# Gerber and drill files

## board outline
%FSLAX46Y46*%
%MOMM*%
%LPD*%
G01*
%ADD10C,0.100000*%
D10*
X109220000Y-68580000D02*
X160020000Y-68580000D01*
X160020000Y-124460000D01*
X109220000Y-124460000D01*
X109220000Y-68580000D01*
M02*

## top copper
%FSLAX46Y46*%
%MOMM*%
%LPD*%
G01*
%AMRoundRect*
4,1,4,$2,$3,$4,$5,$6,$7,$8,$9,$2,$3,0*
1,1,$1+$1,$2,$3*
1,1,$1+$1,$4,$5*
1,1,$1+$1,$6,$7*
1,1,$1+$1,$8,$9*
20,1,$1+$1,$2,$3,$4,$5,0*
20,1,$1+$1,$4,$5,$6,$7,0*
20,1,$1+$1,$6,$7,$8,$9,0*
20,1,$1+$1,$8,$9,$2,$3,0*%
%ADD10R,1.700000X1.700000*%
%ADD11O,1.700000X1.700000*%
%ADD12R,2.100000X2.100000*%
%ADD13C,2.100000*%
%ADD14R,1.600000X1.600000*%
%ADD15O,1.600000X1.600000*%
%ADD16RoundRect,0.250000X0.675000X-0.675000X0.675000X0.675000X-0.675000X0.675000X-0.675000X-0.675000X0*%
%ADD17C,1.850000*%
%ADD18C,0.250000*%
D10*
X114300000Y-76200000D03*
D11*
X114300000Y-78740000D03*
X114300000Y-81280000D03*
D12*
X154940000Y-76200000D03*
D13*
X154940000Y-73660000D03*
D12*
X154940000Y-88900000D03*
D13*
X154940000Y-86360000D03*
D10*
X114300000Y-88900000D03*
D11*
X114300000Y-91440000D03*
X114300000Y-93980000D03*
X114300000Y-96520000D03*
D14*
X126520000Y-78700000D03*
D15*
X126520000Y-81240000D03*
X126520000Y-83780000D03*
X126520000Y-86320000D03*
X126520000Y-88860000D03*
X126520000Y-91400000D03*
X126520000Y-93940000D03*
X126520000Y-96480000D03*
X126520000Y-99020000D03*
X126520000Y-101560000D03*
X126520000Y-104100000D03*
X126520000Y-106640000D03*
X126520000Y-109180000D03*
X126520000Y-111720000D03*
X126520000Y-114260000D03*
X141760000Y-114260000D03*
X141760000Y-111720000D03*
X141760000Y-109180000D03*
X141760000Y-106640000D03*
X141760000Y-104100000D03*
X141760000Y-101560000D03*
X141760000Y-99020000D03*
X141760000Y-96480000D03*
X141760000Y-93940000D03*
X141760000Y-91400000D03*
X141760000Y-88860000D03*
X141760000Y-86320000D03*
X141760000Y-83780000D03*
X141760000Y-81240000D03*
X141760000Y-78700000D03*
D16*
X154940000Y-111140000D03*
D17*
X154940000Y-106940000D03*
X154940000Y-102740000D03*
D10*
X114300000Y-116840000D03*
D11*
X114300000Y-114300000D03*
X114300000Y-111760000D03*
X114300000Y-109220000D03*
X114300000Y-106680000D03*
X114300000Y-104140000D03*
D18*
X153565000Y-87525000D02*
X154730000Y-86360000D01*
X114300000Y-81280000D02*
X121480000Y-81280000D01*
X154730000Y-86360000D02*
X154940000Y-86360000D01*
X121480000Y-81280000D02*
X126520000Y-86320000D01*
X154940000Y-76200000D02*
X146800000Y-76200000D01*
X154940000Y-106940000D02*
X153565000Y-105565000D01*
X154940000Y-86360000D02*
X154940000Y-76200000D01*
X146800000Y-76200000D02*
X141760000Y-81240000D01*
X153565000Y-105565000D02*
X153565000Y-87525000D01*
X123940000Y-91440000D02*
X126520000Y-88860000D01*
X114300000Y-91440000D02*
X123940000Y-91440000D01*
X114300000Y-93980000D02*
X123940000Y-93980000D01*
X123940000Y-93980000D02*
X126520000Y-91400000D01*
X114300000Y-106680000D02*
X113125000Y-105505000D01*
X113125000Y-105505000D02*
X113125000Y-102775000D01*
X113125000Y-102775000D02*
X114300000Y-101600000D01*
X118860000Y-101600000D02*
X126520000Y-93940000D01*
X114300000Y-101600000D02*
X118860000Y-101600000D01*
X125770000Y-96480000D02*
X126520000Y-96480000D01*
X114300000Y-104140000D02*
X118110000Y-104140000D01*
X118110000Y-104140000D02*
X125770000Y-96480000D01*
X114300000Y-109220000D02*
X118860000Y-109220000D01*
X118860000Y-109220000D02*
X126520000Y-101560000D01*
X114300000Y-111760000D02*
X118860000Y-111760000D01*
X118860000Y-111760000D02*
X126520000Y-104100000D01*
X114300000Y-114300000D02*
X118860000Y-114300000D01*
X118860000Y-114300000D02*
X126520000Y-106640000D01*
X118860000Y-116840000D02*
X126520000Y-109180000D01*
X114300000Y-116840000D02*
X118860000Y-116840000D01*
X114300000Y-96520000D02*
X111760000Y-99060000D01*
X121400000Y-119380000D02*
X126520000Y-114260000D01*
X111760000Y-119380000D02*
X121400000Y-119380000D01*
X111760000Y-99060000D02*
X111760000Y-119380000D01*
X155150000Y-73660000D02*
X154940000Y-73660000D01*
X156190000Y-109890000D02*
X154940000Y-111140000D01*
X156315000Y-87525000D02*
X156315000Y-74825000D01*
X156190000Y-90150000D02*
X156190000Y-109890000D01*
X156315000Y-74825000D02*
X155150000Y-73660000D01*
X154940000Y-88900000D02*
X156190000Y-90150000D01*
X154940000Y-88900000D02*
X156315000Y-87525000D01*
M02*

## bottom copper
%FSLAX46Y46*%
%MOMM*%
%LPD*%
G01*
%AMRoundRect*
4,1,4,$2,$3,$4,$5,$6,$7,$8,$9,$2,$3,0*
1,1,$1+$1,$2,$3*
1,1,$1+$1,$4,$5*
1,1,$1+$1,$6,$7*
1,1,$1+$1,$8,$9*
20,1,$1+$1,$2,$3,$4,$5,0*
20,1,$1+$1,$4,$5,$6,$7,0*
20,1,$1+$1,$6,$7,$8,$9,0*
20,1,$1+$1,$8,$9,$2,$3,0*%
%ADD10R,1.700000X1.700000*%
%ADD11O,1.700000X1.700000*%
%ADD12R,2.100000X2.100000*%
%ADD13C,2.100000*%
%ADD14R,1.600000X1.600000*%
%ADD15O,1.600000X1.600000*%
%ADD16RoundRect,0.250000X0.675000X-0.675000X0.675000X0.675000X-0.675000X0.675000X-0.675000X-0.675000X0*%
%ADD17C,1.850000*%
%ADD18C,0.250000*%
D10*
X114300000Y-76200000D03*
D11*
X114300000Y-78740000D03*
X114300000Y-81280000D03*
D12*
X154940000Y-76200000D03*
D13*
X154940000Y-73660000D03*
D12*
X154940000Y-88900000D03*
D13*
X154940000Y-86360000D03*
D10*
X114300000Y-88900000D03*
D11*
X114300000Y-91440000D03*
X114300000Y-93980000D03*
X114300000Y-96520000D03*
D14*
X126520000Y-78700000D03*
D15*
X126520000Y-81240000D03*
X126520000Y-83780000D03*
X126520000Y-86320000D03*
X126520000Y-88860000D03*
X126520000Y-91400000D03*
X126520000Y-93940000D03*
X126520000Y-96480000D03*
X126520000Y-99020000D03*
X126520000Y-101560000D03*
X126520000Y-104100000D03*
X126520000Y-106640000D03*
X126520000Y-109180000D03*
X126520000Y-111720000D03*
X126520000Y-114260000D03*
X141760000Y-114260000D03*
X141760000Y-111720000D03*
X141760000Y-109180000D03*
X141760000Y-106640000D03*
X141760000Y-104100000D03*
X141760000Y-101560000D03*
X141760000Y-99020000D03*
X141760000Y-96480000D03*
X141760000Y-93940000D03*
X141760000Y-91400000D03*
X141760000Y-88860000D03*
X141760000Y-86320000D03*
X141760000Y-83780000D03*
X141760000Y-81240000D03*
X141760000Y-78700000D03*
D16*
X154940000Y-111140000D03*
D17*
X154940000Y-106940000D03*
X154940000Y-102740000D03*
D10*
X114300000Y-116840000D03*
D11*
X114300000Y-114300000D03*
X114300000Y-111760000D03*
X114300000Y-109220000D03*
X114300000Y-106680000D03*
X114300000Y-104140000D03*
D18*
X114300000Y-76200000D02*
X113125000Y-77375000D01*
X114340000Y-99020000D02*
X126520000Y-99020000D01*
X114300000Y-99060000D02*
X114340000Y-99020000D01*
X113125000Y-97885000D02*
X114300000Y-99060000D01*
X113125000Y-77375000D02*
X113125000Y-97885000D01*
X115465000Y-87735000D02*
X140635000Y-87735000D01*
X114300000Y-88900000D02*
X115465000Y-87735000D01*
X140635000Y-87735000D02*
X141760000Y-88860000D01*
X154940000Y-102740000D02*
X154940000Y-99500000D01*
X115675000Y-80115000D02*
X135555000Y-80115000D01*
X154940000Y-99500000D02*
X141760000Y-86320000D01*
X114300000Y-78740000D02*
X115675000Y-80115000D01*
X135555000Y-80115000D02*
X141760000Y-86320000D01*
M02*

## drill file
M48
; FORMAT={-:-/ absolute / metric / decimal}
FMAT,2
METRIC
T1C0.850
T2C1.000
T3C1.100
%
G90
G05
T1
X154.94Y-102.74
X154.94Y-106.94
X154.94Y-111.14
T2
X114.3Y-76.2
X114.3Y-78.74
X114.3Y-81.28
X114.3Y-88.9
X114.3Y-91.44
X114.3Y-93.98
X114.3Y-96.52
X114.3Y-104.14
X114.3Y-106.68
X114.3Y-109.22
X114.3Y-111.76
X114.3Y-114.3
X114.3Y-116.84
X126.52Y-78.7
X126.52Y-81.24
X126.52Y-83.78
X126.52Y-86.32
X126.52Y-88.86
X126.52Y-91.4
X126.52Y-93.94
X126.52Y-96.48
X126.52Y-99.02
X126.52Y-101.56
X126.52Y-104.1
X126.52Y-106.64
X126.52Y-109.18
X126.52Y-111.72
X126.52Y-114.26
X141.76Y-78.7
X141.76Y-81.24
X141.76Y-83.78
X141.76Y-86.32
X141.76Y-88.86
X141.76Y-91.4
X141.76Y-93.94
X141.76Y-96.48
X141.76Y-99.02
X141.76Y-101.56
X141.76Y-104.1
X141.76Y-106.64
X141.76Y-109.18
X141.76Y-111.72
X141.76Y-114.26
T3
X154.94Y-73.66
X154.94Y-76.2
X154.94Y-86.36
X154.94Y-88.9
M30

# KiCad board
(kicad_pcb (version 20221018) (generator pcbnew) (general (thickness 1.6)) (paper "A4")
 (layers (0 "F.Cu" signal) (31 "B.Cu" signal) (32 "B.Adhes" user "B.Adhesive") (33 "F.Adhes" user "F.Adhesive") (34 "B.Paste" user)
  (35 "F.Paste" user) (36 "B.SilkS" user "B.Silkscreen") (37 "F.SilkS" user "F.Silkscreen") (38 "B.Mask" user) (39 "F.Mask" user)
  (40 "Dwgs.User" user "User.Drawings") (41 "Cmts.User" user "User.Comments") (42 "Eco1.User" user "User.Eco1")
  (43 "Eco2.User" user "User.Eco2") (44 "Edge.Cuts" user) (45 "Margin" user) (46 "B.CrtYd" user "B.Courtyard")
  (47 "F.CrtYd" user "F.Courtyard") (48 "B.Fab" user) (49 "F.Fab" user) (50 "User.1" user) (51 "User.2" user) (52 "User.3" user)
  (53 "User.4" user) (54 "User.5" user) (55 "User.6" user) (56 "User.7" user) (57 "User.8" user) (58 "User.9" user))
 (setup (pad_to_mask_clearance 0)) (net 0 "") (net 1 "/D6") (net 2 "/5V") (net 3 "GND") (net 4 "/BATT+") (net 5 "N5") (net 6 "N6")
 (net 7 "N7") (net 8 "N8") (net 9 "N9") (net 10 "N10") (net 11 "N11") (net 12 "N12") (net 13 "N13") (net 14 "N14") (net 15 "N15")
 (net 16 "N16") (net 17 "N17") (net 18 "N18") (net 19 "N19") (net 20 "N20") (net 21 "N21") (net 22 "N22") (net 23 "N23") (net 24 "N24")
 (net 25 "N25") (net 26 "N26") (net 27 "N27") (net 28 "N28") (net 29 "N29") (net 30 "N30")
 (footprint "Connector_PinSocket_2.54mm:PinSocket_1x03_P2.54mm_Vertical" (layer "F.Cu") (at 114.3 76.2)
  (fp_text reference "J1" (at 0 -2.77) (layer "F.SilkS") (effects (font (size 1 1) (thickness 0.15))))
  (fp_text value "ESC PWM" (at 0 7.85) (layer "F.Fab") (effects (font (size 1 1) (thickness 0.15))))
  (pad "1" thru_hole rect (at 0 0) (size 1.7 1.7) (drill 1) (layers "*.Cu" "*.Mask") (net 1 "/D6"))
  (pad "2" thru_hole oval (at 0 2.54) (size 1.7 1.7) (drill 1) (layers "*.Cu" "*.Mask") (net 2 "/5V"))
  (pad "3" thru_hole oval (at 0 5.08) (size 1.7 1.7) (drill 1) (layers "*.Cu" "*.Mask") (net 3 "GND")))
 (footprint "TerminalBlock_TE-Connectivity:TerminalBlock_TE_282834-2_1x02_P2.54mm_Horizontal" (layer "F.Cu") (at 154.94 76.2 90)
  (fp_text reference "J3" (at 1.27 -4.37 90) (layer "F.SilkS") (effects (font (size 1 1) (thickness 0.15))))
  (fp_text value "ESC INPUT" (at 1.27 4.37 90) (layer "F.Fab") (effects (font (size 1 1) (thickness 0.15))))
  (pad "1" thru_hole rect (at 0 0 90) (size 2.1 2.1) (drill 1.1) (layers "*.Cu" "*.Mask") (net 3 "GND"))
  (pad "2" thru_hole circle (at 2.54 0 90) (size 2.1 2.1) (drill 1.1) (layers "*.Cu" "*.Mask") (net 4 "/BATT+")))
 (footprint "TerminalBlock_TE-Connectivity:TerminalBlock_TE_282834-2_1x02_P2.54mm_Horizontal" (layer "F.Cu") (at 154.94 88.9 90)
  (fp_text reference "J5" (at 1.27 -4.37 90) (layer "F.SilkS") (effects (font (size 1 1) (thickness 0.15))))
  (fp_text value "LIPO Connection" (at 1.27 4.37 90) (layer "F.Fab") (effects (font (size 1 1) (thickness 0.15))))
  (pad "1" thru_hole rect (at 0 0 90) (size 2.1 2.1) (drill 1.1) (layers "*.Cu" "*.Mask") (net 4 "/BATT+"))
  (pad "2" thru_hole circle (at 2.54 0 90) (size 2.1 2.1) (drill 1.1) (layers "*.Cu" "*.Mask") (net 3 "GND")))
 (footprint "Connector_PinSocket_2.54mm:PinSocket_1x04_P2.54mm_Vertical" (layer "F.Cu") (at 114.3 88.9)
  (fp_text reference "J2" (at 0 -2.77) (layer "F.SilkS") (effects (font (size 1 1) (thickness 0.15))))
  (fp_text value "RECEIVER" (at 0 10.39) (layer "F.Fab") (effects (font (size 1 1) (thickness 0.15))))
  (pad "1" thru_hole rect (at 0 0) (size 1.7 1.7) (drill 1) (layers "*.Cu" "*.Mask") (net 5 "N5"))
  (pad "2" thru_hole oval (at 0 2.54) (size 1.7 1.7) (drill 1) (layers "*.Cu" "*.Mask") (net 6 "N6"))
  (pad "3" thru_hole oval (at 0 5.08) (size 1.7 1.7) (drill 1) (layers "*.Cu" "*.Mask") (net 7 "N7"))
  (pad "4" thru_hole oval (at 0 7.62) (size 1.7 1.7) (drill 1) (layers "*.Cu" "*.Mask") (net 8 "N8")))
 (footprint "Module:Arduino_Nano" (layer "F.Cu") (at 126.52 78.7)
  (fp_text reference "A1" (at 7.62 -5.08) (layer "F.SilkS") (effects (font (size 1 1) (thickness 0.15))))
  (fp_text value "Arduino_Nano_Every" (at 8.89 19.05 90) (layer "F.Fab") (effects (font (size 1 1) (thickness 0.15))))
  (pad "1" thru_hole rect (at 0 0) (size 1.6 1.6) (drill 1) (layers "*.Cu" "*.Mask") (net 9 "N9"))
  (pad "2" thru_hole oval (at 0 2.54) (size 1.6 1.6) (drill 1) (layers "*.Cu" "*.Mask") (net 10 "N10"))
  (pad "3" thru_hole oval (at 0 5.08) (size 1.6 1.6) (drill 1) (layers "*.Cu" "*.Mask") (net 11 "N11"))
  (pad "4" thru_hole oval (at 0 7.62) (size 1.6 1.6) (drill 1) (layers "*.Cu" "*.Mask") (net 3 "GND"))
  (pad "5" thru_hole oval (at 0 10.16) (size 1.6 1.6) (drill 1) (layers "*.Cu" "*.Mask") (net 6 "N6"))
  (pad "6" thru_hole oval (at 0 12.7) (size 1.6 1.6) (drill 1) (layers "*.Cu" "*.Mask") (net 7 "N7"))
  (pad "7" thru_hole oval (at 0 15.24) (size 1.6 1.6) (drill 1) (layers "*.Cu" "*.Mask") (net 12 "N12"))
  (pad "8" thru_hole oval (at 0 17.78) (size 1.6 1.6) (drill 1) (layers "*.Cu" "*.Mask") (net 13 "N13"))
  (pad "9" thru_hole oval (at 0 20.32) (size 1.6 1.6) (drill 1) (layers "*.Cu" "*.Mask") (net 1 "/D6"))
  (pad "10" thru_hole oval (at 0 22.86) (size 1.6 1.6) (drill 1) (layers "*.Cu" "*.Mask") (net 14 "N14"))
  (pad "11" thru_hole oval (at 0 25.4) (size 1.6 1.6) (drill 1) (layers "*.Cu" "*.Mask") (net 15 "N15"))
  (pad "12" thru_hole oval (at 0 27.94) (size 1.6 1.6) (drill 1) (layers "*.Cu" "*.Mask") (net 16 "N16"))
  (pad "13" thru_hole oval (at 0 30.48) (size 1.6 1.6) (drill 1) (layers "*.Cu" "*.Mask") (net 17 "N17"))
  (pad "14" thru_hole oval (at 0 33.02) (size 1.6 1.6) (drill 1) (layers "*.Cu" "*.Mask") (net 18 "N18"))
  (pad "15" thru_hole oval (at 0 35.56) (size 1.6 1.6) (drill 1) (layers "*.Cu" "*.Mask") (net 8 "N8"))
  (pad "16" thru_hole oval (at 15.24 35.56) (size 1.6 1.6) (drill 1) (layers "*.Cu" "*.Mask") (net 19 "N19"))
  (pad "17" thru_hole oval (at 15.24 33.02) (size 1.6 1.6) (drill 1) (layers "*.Cu" "*.Mask") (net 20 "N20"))
  (pad "18" thru_hole oval (at 15.24 30.48) (size 1.6 1.6) (drill 1) (layers "*.Cu" "*.Mask") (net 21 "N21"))
  (pad "19" thru_hole oval (at 15.24 27.94) (size 1.6 1.6) (drill 1) (layers "*.Cu" "*.Mask") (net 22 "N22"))
  (pad "20" thru_hole oval (at 15.24 25.4) (size 1.6 1.6) (drill 1) (layers "*.Cu" "*.Mask") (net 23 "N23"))
  (pad "21" thru_hole oval (at 15.24 22.86) (size 1.6 1.6) (drill 1) (layers "*.Cu" "*.Mask") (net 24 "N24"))
  (pad "22" thru_hole oval (at 15.24 20.32) (size 1.6 1.6) (drill 1) (layers "*.Cu" "*.Mask") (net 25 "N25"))
  (pad "23" thru_hole oval (at 15.24 17.78) (size 1.6 1.6) (drill 1) (layers "*.Cu" "*.Mask") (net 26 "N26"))
  (pad "24" thru_hole oval (at 15.24 15.24) (size 1.6 1.6) (drill 1) (layers "*.Cu" "*.Mask") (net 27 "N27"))
  (pad "25" thru_hole oval (at 15.24 12.7) (size 1.6 1.6) (drill 1) (layers "*.Cu" "*.Mask") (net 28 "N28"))
  (pad "26" thru_hole oval (at 15.24 10.16) (size 1.6 1.6) (drill 1) (layers "*.Cu" "*.Mask") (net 5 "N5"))
  (pad "27" thru_hole oval (at 15.24 7.62) (size 1.6 1.6) (drill 1) (layers "*.Cu" "*.Mask") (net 2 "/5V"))
  (pad "28" thru_hole oval (at 15.24 5.08) (size 1.6 1.6) (drill 1) (layers "*.Cu" "*.Mask") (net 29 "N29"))
  (pad "29" thru_hole oval (at 15.24 2.54) (size 1.6 1.6) (drill 1) (layers "*.Cu" "*.Mask") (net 3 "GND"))
  (pad "30" thru_hole oval (at 15.24 0) (size 1.6 1.6) (drill 1) (layers "*.Cu" "*.Mask") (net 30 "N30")))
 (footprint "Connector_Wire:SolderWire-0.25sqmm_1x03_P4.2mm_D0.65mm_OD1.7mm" (layer "F.Cu") (at 154.94 111.14 90)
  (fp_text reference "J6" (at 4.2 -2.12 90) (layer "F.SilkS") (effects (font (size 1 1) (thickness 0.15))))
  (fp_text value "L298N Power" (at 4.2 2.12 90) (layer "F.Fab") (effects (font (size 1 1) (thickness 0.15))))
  (pad "1" thru_hole roundrect (at 0 0 90) (size 1.85 1.85) (drill 0.85) (layers "*.Cu" "*.Mask") (roundrect_rratio 0.1351351351)
   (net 4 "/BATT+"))
  (pad "2" thru_hole circle (at 4.2 0 90) (size 1.85 1.85) (drill 0.85) (layers "*.Cu" "*.Mask") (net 3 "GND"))
  (pad "3" thru_hole circle (at 8.4 0 90) (size 1.85 1.85) (drill 0.85) (layers "*.Cu" "*.Mask") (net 2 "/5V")))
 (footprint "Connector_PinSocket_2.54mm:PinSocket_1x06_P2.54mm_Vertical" (layer "F.Cu") (at 114.3 116.84 180)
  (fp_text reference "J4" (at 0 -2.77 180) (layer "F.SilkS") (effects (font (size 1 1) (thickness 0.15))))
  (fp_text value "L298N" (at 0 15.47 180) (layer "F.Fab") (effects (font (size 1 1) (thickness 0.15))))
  (pad "1" thru_hole rect (at 0 0 180) (size 1.7 1.7) (drill 1) (layers "*.Cu" "*.Mask") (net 17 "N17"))
  (pad "2" thru_hole oval (at 0 2.54 180) (size 1.7 1.7) (drill 1) (layers "*.Cu" "*.Mask") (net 16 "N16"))
  (pad "3" thru_hole oval (at 0 5.08 180) (size 1.7 1.7) (drill 1) (layers "*.Cu" "*.Mask") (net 15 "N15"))
  (pad "4" thru_hole oval (at 0 7.62 180) (size 1.7 1.7) (drill 1) (layers "*.Cu" "*.Mask") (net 14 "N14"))
  (pad "5" thru_hole oval (at 0 10.16 180) (size 1.7 1.7) (drill 1) (layers "*.Cu" "*.Mask") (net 12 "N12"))
  (pad "6" thru_hole oval (at 0 12.7 180) (size 1.7 1.7) (drill 1) (layers "*.Cu" "*.Mask") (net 13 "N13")))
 (gr_rect (start 109.22 68.58) (end 160.02 124.46) (stroke (width 0.1) (type default)) (fill none) (layer "Edge.Cuts"))
 (segment (start 153.565 87.525) (end 154.73 86.36) (width 0.25) (layer "F.Cu") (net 3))
 (segment (start 114.3 81.28) (end 121.48 81.28) (width 0.25) (layer "F.Cu") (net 3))
 (segment (start 154.73 86.36) (end 154.94 86.36) (width 0.25) (layer "F.Cu") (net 3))
 (segment (start 121.48 81.28) (end 126.52 86.32) (width 0.25) (layer "F.Cu") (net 3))
 (segment (start 154.94 76.2) (end 146.8 76.2) (width 0.25) (layer "F.Cu") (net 3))
 (segment (start 154.94 106.94) (end 153.565 105.565) (width 0.25) (layer "F.Cu") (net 3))
 (segment (start 154.94 86.36) (end 154.94 76.2) (width 0.25) (layer "F.Cu") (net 3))
 (segment (start 146.8 76.2) (end 141.76 81.24) (width 0.25) (layer "F.Cu") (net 3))
 (segment (start 153.565 105.565) (end 153.565 87.525) (width 0.25) (layer "F.Cu") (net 3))
 (segment (start 123.94 91.44) (end 126.52 88.86) (width 0.25) (layer "F.Cu") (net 6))
 (segment (start 114.3 91.44) (end 123.94 91.44) (width 0.25) (layer "F.Cu") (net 6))
 (segment (start 114.3 93.98) (end 123.94 93.98) (width 0.25) (layer "F.Cu") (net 7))
 (segment (start 123.94 93.98) (end 126.52 91.4) (width 0.25) (layer "F.Cu") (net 7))
 (segment (start 114.3 106.68) (end 113.125 105.505) (width 0.25) (layer "F.Cu") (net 12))
 (segment (start 113.125 105.505) (end 113.125 102.775) (width 0.25) (layer "F.Cu") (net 12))
 (segment (start 113.125 102.775) (end 114.3 101.6) (width 0.25) (layer "F.Cu") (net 12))
 (segment (start 118.86 101.6) (end 126.52 93.94) (width 0.25) (layer "F.Cu") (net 12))
 (segment (start 114.3 101.6) (end 118.86 101.6) (width 0.25) (layer "F.Cu") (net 12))
 (segment (start 125.77 96.48) (end 126.52 96.48) (width 0.25) (layer "F.Cu") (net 13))
 (segment (start 114.3 104.14) (end 118.11 104.14) (width 0.25) (layer "F.Cu") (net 13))
 (segment (start 118.11 104.14) (end 125.77 96.48) (width 0.25) (layer "F.Cu") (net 13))
 (segment (start 114.3 76.2) (end 113.125 77.375) (width 0.25) (layer "B.Cu") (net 1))
 (segment (start 114.34 99.02) (end 126.52 99.02) (width 0.25) (layer "B.Cu") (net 1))
 (segment (start 114.3 99.06) (end 114.34 99.02) (width 0.25) (layer "B.Cu") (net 1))
 (segment (start 113.125 97.885) (end 114.3 99.06) (width 0.25) (layer "B.Cu") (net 1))
 (segment (start 113.125 77.375) (end 113.125 97.885) (width 0.25) (layer "B.Cu") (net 1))
 (segment (start 114.3 109.22) (end 118.86 109.22) (width 0.25) (layer "F.Cu") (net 14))
 (segment (start 118.86 109.22) (end 126.52 101.56) (width 0.25) (layer "F.Cu") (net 14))
 (segment (start 114.3 111.76) (end 118.86 111.76) (width 0.25) (layer "F.Cu") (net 15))
 (segment (start 118.86 111.76) (end 126.52 104.1) (width 0.25) (layer "F.Cu") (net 15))
 (segment (start 114.3 114.3) (end 118.86 114.3) (width 0.25) (layer "F.Cu") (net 16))
 (segment (start 118.86 114.3) (end 126.52 106.64) (width 0.25) (layer "F.Cu") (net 16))
 (segment (start 118.86 116.84) (end 126.52 109.18) (width 0.25) (layer "F.Cu") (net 17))
 (segment (start 114.3 116.84) (end 118.86 116.84) (width 0.25) (layer "F.Cu") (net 17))
 (segment (start 114.3 96.52) (end 111.76 99.06) (width 0.25) (layer "F.Cu") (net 8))
 (segment (start 121.4 119.38) (end 126.52 114.26) (width 0.25) (layer "F.Cu") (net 8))
 (segment (start 111.76 119.38) (end 121.4 119.38) (width 0.25) (layer "F.Cu") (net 8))
 (segment (start 111.76 99.06) (end 111.76 119.38) (width 0.25) (layer "F.Cu") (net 8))
 (segment (start 115.465 87.735) (end 140.635 87.735) (width 0.25) (layer "B.Cu") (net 5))
 (segment (start 114.3 88.9) (end 115.465 87.735) (width 0.25) (layer "B.Cu") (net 5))
 (segment (start 140.635 87.735) (end 141.76 88.86) (width 0.25) (layer "B.Cu") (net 5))
 (segment (start 154.94 102.74) (end 154.94 99.5) (width 0.25) (layer "B.Cu") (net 2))
 (segment (start 115.675 80.115) (end 135.555 80.115) (width 0.25) (layer "B.Cu") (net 2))
 (segment (start 154.94 99.5) (end 141.76 86.32) (width 0.25) (layer "B.Cu") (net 2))
 (segment (start 114.3 78.74) (end 115.675 80.115) (width 0.25) (layer "B.Cu") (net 2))
 (segment (start 135.555 80.115) (end 141.76 86.32) (width 0.25) (layer "B.Cu") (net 2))
 (segment (start 155.15 73.66) (end 154.94 73.66) (width 0.25) (layer "F.Cu") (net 4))
 (segment (start 156.19 109.89) (end 154.94 111.14) (width 0.25) (layer "F.Cu") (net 4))
 (segment (start 156.315 87.525) (end 156.315 74.825) (width 0.25) (layer "F.Cu") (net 4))
 (segment (start 156.19 90.15) (end 156.19 109.89) (width 0.25) (layer "F.Cu") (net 4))
 (segment (start 156.315 74.825) (end 155.15 73.66) (width 0.25) (layer "F.Cu") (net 4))
 (segment (start 154.94 88.9) (end 156.19 90.15) (width 0.25) (layer "F.Cu") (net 4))
 (segment (start 154.94 88.9) (end 156.315 87.525) (width 0.25) (layer "F.Cu") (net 4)))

